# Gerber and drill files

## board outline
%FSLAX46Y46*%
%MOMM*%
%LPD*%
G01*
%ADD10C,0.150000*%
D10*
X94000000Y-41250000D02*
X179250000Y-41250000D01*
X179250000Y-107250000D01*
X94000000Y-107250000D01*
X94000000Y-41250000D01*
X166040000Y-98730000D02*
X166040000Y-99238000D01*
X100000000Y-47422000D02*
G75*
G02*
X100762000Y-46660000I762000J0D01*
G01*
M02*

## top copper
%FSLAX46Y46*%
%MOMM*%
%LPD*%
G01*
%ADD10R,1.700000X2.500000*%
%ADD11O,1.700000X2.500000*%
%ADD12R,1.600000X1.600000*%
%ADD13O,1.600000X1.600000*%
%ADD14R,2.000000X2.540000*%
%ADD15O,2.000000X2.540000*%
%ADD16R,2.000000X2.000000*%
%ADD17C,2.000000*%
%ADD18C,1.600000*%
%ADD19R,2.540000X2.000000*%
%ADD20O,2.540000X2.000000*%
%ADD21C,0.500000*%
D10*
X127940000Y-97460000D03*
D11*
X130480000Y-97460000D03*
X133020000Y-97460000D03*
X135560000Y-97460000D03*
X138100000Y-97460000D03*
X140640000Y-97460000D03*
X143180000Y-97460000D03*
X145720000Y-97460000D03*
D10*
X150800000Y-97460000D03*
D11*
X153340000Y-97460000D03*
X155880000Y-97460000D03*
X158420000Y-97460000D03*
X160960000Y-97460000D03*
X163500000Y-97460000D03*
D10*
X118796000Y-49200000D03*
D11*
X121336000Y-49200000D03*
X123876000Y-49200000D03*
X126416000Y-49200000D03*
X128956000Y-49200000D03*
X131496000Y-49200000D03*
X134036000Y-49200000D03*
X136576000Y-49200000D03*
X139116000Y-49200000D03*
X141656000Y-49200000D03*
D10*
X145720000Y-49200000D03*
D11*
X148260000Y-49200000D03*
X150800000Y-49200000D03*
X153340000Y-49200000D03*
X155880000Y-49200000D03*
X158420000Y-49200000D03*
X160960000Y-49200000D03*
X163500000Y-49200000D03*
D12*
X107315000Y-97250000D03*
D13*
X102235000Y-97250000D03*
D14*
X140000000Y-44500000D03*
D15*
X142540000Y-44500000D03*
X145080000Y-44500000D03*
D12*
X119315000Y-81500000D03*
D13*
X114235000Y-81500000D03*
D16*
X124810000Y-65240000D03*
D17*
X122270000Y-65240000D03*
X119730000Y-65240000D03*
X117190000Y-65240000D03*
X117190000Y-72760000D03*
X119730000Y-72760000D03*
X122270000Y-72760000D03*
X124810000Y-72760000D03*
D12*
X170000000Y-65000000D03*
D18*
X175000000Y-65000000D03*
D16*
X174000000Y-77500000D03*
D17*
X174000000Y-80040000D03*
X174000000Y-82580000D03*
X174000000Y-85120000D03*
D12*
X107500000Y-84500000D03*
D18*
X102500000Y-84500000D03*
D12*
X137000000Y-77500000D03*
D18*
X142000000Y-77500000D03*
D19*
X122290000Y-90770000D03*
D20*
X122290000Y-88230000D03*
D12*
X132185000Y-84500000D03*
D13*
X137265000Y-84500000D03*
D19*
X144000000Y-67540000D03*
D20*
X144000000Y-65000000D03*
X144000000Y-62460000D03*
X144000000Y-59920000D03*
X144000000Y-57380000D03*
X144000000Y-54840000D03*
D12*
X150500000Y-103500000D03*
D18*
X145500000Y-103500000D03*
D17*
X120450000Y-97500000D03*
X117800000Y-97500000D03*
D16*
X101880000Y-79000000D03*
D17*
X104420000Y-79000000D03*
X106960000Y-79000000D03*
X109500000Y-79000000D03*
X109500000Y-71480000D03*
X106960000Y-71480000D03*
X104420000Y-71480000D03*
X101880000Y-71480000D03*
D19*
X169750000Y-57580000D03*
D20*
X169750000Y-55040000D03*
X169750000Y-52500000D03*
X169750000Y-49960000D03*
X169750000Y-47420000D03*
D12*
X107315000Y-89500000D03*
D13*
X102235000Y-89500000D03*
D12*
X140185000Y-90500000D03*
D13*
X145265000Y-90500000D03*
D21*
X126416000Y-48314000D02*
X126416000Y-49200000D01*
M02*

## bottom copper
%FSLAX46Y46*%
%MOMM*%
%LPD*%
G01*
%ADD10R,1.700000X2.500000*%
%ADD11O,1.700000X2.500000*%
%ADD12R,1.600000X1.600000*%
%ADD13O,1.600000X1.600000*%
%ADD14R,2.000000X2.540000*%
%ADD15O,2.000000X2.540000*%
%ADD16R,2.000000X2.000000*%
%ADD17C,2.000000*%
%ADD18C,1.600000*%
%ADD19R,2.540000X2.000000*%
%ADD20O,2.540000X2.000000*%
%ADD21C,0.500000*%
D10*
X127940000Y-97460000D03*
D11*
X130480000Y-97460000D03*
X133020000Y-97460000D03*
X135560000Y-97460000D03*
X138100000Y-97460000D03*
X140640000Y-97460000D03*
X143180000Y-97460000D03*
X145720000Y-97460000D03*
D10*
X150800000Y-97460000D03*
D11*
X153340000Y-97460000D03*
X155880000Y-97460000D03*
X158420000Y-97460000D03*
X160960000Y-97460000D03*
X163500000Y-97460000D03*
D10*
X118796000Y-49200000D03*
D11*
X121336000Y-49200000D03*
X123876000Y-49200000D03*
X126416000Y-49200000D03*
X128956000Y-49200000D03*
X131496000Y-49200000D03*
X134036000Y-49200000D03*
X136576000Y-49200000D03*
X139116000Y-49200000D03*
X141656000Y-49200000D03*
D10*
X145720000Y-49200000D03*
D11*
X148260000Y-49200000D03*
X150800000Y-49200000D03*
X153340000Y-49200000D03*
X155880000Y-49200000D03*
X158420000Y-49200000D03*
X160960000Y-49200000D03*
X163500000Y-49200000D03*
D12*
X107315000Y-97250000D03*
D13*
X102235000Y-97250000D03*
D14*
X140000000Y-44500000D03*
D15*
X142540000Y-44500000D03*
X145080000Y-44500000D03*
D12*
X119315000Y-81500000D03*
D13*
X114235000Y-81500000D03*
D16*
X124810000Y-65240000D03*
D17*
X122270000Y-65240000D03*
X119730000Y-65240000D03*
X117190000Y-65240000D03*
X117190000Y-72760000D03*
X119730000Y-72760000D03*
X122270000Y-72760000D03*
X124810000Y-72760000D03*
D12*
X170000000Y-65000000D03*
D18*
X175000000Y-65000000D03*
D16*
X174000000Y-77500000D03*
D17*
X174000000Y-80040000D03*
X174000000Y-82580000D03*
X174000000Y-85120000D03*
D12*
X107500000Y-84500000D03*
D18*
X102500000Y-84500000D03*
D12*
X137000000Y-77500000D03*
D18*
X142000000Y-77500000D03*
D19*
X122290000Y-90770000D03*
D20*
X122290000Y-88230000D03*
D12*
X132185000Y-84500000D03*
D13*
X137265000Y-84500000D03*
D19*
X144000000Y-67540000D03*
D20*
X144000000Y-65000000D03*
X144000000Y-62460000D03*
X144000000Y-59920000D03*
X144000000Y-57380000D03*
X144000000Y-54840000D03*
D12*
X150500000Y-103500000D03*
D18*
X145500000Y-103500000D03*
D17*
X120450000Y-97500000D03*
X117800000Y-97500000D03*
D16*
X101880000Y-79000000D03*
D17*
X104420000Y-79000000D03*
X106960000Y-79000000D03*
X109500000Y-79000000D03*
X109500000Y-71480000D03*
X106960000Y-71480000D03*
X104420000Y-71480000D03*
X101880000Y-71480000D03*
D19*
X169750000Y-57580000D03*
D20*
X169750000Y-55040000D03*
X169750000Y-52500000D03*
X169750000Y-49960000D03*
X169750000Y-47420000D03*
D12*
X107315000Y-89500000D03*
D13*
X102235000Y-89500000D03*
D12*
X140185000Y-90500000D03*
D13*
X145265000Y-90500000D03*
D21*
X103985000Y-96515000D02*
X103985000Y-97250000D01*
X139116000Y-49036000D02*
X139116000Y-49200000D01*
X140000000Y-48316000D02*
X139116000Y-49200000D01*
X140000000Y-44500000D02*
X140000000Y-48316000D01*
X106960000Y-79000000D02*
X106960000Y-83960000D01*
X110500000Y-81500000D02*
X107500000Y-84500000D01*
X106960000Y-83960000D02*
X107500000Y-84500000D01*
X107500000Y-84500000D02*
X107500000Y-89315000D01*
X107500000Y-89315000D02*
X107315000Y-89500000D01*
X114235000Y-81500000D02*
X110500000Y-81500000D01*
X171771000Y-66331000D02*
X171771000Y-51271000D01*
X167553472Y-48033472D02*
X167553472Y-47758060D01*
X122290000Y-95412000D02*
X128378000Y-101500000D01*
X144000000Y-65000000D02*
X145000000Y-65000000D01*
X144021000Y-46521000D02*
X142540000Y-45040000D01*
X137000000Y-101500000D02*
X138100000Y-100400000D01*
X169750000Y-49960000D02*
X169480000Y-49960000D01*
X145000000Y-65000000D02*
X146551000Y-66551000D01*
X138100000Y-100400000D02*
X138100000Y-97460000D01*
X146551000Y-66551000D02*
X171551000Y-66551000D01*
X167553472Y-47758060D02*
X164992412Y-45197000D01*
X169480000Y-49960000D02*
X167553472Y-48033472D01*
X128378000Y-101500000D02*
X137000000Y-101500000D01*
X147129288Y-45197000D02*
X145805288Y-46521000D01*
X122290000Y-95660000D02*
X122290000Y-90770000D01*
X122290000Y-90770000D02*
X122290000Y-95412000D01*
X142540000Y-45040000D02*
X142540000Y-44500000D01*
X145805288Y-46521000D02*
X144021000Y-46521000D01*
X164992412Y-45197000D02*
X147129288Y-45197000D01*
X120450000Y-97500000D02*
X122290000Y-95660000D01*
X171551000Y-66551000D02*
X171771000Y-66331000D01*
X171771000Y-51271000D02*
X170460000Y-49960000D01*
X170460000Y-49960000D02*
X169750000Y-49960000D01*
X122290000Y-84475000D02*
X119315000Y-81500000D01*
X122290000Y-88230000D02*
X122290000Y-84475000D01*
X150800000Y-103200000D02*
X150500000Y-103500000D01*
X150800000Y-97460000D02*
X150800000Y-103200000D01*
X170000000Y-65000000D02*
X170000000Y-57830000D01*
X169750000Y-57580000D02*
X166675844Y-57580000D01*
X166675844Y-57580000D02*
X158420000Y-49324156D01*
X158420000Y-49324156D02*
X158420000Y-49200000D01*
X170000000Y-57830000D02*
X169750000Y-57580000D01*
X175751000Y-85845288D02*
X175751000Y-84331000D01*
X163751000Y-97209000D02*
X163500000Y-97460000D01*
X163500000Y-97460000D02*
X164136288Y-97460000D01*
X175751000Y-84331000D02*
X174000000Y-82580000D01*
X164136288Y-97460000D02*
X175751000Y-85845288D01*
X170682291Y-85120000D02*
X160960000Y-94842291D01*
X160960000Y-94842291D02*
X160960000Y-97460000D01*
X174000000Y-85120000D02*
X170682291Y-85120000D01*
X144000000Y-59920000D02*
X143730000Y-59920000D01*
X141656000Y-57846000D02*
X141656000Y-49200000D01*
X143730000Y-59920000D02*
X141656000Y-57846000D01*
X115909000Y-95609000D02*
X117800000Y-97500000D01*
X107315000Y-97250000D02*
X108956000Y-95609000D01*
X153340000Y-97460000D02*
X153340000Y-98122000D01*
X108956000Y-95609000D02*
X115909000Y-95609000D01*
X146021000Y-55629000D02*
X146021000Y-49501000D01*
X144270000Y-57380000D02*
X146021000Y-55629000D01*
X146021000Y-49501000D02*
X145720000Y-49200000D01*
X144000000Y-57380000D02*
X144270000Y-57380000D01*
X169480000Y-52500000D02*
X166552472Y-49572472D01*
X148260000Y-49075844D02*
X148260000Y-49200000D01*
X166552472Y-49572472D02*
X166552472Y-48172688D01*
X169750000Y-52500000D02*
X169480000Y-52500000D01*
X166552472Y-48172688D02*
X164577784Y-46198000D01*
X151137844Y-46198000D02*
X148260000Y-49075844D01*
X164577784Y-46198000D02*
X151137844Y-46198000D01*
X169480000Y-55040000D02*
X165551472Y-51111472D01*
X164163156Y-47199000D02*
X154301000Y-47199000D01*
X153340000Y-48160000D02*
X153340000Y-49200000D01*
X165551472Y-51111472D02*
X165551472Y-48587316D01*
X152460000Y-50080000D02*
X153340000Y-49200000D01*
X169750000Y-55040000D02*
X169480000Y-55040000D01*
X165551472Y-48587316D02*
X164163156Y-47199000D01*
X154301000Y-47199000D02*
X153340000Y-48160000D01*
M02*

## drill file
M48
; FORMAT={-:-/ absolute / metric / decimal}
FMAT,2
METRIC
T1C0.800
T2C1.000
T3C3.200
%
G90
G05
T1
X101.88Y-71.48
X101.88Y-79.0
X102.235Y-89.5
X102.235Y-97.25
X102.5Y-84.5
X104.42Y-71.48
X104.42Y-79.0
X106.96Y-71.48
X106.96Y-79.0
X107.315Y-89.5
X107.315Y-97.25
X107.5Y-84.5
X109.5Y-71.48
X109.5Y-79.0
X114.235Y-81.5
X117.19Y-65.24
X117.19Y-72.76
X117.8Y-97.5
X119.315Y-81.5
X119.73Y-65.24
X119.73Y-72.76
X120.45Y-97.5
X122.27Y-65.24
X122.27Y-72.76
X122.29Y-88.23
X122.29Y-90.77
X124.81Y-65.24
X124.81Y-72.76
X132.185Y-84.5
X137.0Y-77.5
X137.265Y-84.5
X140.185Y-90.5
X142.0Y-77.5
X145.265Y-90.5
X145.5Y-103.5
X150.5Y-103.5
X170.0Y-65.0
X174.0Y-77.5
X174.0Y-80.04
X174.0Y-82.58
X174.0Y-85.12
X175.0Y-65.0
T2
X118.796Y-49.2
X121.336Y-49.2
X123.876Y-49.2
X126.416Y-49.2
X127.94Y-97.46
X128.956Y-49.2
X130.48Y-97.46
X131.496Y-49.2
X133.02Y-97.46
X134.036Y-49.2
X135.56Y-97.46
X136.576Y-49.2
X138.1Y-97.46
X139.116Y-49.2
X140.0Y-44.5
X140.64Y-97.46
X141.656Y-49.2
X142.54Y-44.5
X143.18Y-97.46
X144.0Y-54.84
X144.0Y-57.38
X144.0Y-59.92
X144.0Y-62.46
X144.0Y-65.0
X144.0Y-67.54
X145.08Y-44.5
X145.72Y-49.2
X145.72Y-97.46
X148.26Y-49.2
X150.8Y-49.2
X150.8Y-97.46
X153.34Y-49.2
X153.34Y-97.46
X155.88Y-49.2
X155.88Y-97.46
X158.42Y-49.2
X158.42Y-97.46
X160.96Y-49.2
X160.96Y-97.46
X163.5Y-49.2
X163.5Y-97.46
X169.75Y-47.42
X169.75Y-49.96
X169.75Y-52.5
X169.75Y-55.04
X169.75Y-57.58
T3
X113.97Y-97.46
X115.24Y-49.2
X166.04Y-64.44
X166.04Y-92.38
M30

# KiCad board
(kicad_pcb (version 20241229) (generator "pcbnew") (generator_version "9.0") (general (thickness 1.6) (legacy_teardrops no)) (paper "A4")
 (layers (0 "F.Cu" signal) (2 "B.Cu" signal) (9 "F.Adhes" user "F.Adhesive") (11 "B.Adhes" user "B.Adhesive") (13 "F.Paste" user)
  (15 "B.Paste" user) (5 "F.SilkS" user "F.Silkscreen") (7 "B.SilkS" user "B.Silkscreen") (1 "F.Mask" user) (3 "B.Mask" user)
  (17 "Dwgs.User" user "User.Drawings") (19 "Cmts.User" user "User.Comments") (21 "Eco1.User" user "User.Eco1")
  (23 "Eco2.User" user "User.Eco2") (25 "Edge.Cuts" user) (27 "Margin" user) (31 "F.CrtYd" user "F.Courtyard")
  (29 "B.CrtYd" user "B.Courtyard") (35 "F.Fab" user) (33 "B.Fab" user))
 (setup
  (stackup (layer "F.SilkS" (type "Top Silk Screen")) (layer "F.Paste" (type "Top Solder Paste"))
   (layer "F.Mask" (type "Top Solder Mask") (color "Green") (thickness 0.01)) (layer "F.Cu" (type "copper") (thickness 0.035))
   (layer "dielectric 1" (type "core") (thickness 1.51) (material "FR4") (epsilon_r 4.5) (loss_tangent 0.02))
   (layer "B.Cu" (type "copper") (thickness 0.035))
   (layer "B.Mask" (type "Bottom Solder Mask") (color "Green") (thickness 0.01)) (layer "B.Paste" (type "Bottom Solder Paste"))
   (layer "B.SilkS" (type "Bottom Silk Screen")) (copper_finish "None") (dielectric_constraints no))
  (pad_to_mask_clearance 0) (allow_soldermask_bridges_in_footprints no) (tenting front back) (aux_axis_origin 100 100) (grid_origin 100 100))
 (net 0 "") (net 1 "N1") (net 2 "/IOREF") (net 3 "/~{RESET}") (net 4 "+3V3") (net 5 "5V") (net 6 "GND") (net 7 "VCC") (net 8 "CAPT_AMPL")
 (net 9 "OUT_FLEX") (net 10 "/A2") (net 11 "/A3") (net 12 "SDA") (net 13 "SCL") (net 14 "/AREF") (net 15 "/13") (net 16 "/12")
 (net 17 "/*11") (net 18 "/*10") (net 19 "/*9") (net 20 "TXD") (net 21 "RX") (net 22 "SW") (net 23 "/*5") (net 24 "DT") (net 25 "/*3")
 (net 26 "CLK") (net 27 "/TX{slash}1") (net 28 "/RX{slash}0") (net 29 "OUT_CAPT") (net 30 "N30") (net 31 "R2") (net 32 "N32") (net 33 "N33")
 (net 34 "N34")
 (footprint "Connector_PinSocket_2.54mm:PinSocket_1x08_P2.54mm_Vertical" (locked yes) (layer "F.Cu") (at 127.94 97.46 90)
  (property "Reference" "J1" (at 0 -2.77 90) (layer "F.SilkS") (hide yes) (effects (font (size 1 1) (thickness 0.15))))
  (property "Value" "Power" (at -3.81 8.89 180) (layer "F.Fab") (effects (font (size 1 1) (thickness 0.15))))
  (pad "1" thru_hole rect (at 0 0 90) (size 2.5 1.7) (drill 1) (layers "*.Cu" "*.Mask") (remove_unused_layers no) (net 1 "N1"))
  (pad "2" thru_hole oval (at 0 2.54 90) (size 2.5 1.7) (drill 1) (layers "*.Cu" "*.Mask") (remove_unused_layers no) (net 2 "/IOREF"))
  (pad "3" thru_hole oval (at 0 5.08 90) (size 2.5 1.7) (drill 1) (layers "*.Cu" "*.Mask") (remove_unused_layers no) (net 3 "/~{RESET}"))
  (pad "4" thru_hole oval (at 0 7.62 90) (size 2.5 1.7) (drill 1) (layers "*.Cu" "*.Mask") (remove_unused_layers no) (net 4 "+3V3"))
  (pad "5" thru_hole oval (at 0 10.16 90) (size 2.5 1.7) (drill 1) (layers "*.Cu" "*.Mask") (remove_unused_layers no) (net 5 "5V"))
  (pad "6" thru_hole oval (at 0 12.7 90) (size 2.5 1.7) (drill 1) (layers "*.Cu" "*.Mask") (remove_unused_layers no) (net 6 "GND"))
  (pad "7" thru_hole oval (at 0 15.24 90) (size 2.5 1.7) (drill 1) (layers "*.Cu" "*.Mask") (remove_unused_layers no) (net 6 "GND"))
  (pad "8" thru_hole oval (at 0 17.78 90) (size 2.5 1.7) (drill 1) (layers "*.Cu" "*.Mask") (remove_unused_layers no) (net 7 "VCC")))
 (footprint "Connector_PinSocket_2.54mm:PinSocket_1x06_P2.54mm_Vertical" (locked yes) (layer "F.Cu") (at 150.8 97.46 90)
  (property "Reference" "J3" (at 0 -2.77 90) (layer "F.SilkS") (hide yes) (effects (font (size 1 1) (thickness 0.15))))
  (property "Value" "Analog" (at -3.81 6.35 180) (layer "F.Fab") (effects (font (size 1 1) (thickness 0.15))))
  (pad "1" thru_hole rect (at 0 0 90) (size 2.5 1.7) (drill 1) (layers "*.Cu" "*.Mask") (remove_unused_layers no) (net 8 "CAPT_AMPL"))
  (pad "2" thru_hole oval (at 0 2.54 90) (size 2.5 1.7) (drill 1) (layers "*.Cu" "*.Mask") (remove_unused_layers no) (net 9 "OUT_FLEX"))
  (pad "3" thru_hole oval (at 0 5.08 90) (size 2.5 1.7) (drill 1) (layers "*.Cu" "*.Mask") (remove_unused_layers no) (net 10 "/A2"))
  (pad "4" thru_hole oval (at 0 7.62 90) (size 2.5 1.7) (drill 1) (layers "*.Cu" "*.Mask") (remove_unused_layers no) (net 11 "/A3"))
  (pad "5" thru_hole oval (at 0 10.16 90) (size 2.5 1.7) (drill 1) (layers "*.Cu" "*.Mask") (remove_unused_layers no) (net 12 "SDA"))
  (pad "6" thru_hole oval (at 0 12.7 90) (size 2.5 1.7) (drill 1) (layers "*.Cu" "*.Mask") (remove_unused_layers no) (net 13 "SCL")))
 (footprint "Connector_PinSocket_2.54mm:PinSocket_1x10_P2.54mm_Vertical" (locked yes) (layer "F.Cu") (at 118.796 49.2 90)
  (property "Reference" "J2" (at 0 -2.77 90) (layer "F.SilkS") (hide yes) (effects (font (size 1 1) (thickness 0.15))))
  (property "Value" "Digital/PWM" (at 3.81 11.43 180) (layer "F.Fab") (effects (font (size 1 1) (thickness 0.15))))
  (pad "1" thru_hole rect (at 0 0 90) (size 2.5 1.7) (drill 1) (layers "*.Cu" "*.Mask") (remove_unused_layers no) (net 13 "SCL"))
  (pad "2" thru_hole oval (at 0 2.54 90) (size 2.5 1.7) (drill 1) (layers "*.Cu" "*.Mask") (remove_unused_layers no) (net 12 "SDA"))
  (pad "3" thru_hole oval (at 0 5.08 90) (size 2.5 1.7) (drill 1) (layers "*.Cu" "*.Mask") (remove_unused_layers no) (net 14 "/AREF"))
  (pad "4" thru_hole oval (at 0 7.62 90) (size 2.5 1.7) (drill 1) (layers "*.Cu" "*.Mask") (remove_unused_layers no) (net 6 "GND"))
  (pad "5" thru_hole oval (at 0 10.16 90) (size 2.5 1.7) (drill 1) (layers "*.Cu" "*.Mask") (remove_unused_layers no) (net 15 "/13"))
  (pad "6" thru_hole oval (at 0 12.7 90) (size 2.5 1.7) (drill 1) (layers "*.Cu" "*.Mask") (remove_unused_layers no) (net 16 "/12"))
  (pad "7" thru_hole oval (at 0 15.24 90) (size 2.5 1.7) (drill 1) (layers "*.Cu" "*.Mask") (remove_unused_layers no) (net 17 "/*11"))
  (pad "8" thru_hole oval (at 0 17.78 90) (size 2.5 1.7) (drill 1) (layers "*.Cu" "*.Mask") (remove_unused_layers no) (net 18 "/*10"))
  (pad "9" thru_hole oval (at 0 20.32 90) (size 2.5 1.7) (drill 1) (layers "*.Cu" "*.Mask") (remove_unused_layers no) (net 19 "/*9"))
  (pad "10" thru_hole oval (at 0 22.86 90) (size 2.5 1.7) (drill 1) (layers "*.Cu" "*.Mask") (remove_unused_layers no) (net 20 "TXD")))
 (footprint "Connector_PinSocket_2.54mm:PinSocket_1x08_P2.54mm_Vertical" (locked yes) (layer "F.Cu") (at 145.72 49.2 90)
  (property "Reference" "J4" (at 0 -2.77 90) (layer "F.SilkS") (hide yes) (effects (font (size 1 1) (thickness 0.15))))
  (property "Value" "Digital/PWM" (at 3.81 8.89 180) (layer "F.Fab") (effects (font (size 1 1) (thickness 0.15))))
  (pad "1" thru_hole rect (at 0 0 90) (size 2.5 1.7) (drill 1) (layers "*.Cu" "*.Mask") (remove_unused_layers no) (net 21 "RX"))
  (pad "2" thru_hole oval (at 0 2.54 90) (size 2.5 1.7) (drill 1) (layers "*.Cu" "*.Mask") (remove_unused_layers no) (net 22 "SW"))
  (pad "3" thru_hole oval (at 0 5.08 90) (size 2.5 1.7) (drill 1) (layers "*.Cu" "*.Mask") (remove_unused_layers no) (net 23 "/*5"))
  (pad "4" thru_hole oval (at 0 7.62 90) (size 2.5 1.7) (drill 1) (layers "*.Cu" "*.Mask") (remove_unused_layers no) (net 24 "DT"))
  (pad "5" thru_hole oval (at 0 10.16 90) (size 2.5 1.7) (drill 1) (layers "*.Cu" "*.Mask") (remove_unused_layers no) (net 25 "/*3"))
  (pad "6" thru_hole oval (at 0 12.7 90) (size 2.5 1.7) (drill 1) (layers "*.Cu" "*.Mask") (remove_unused_layers no) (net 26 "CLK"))
  (pad "7" thru_hole oval (at 0 15.24 90) (size 2.5 1.7) (drill 1) (layers "*.Cu" "*.Mask") (remove_unused_layers no) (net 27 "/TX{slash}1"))
  (pad "8" thru_hole oval (at 0 17.78 90) (size 2.5 1.7) (drill 1) (layers "*.Cu" "*.Mask") (remove_unused_layers no) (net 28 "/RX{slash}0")))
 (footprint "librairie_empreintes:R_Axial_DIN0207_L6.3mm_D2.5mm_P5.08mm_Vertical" (layer "F.Cu") (at 107.315 97.25 180)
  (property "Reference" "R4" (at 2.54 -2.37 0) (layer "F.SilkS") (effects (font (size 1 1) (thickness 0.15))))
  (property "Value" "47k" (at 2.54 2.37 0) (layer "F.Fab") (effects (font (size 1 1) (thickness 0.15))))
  (pad "1" thru_hole rect (at 0 0 180) (size 1.6 1.6) (drill 0.8) (layers "*.Cu" "*.Mask") (remove_unused_layers no) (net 9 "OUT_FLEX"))
  (pad "2" thru_hole oval (at 5.08 0 180) (size 1.6 1.6) (drill 0.8) (layers "*.Cu" "*.Mask") (remove_unused_layers no) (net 6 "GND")))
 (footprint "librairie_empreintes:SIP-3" (layer "F.Cu") (at 142.54 44.5)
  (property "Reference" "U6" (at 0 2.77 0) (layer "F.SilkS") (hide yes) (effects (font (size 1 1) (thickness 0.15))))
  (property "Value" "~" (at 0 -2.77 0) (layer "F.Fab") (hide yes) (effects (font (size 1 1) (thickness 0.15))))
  (pad "1" thru_hole rect (at -2.54 0) (size 2 2.54) (drill 1) (layers "*.Cu" "*.Mask") (remove_unused_layers no) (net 19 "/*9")
   (thermal_bridge_angle 45))
  (pad "2" thru_hole oval (at 0 0) (size 2 2.54) (drill 1) (layers "*.Cu" "*.Mask") (remove_unused_layers no) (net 5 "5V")
   (thermal_bridge_angle 45))
  (pad "3" thru_hole oval (at 2.54 0) (size 2 2.54) (drill 1) (layers "*.Cu" "*.Mask") (remove_unused_layers no) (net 6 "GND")
   (thermal_bridge_angle 45)))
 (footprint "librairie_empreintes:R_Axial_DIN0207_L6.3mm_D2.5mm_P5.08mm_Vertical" (layer "F.Cu") (at 119.315 81.5 180)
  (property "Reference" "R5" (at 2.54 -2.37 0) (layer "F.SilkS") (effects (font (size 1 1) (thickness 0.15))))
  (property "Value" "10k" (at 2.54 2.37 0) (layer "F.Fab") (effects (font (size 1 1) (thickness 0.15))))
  (pad "1" thru_hole rect (at 0 0 180) (size 1.6 1.6) (drill 0.8) (layers "*.Cu" "*.Mask") (remove_unused_layers no) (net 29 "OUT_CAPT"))
  (pad "2" thru_hole oval (at 5.08 0 180) (size 1.6 1.6) (drill 0.8) (layers "*.Cu" "*.Mask") (remove_unused_layers no) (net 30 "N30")))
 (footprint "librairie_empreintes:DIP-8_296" (layer "F.Cu") (at 121 69 180)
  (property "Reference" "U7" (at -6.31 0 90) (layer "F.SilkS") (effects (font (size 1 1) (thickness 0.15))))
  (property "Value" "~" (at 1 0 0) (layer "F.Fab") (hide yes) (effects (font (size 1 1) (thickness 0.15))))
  (pad "1" thru_hole rect (at -3.81 3.76 180) (size 2 2) (drill 0.8) (layers "*.Cu" "*.Mask") (remove_unused_layers no) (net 18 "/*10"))
  (pad "2" thru_hole circle (at -1.27 3.76 180) (size 2 2) (drill 0.8) (layers "*.Cu" "*.Mask") (remove_unused_layers no) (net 15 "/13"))
  (pad "3" thru_hole circle (at 1.27 3.76 180) (size 2 2) (drill 0.8) (layers "*.Cu" "*.Mask") (remove_unused_layers no) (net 17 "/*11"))
  (pad "4" thru_hole circle (at 3.81 3.76 180) (size 2 2) (drill 0.8) (layers "*.Cu" "*.Mask") (remove_unused_layers no) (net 6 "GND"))
  (pad "5" thru_hole circle (at 3.81 -3.76 180) (size 2 2) (drill 0.8) (layers "*.Cu" "*.Mask") (remove_unused_layers no) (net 6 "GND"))
  (pad "6" thru_hole circle (at 1.27 -3.76 180) (size 2 2) (drill 0.8) (layers "*.Cu" "*.Mask") (remove_unused_layers no) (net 6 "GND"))
  (pad "7" thru_hole circle (at -1.27 -3.76 180) (size 2 2) (drill 0.8) (layers "*.Cu" "*.Mask") (remove_unused_layers no) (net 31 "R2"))
  (pad "8" thru_hole circle (at -3.81 -3.76 180) (size 2 2) (drill 0.8) (layers "*.Cu" "*.Mask") (remove_unused_layers no) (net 5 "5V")))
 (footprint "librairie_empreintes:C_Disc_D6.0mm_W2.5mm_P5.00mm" (layer "F.Cu") (at 170 65)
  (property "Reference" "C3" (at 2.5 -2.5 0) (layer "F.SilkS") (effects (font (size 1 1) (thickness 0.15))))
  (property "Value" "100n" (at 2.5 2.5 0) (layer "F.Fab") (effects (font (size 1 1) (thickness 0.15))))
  (pad "1" thru_hole rect (at 0 0) (size 1.6 1.6) (drill 0.8) (layers "*.Cu" "*.Mask") (remove_unused_layers no) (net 26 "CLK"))
  (pad "2" thru_hole circle (at 5 0) (size 1.6 1.6) (drill 0.8) (layers "*.Cu" "*.Mask") (remove_unused_layers no) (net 6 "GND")))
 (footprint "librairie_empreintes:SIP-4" (layer "F.Cu") (at 174 81.31 -90)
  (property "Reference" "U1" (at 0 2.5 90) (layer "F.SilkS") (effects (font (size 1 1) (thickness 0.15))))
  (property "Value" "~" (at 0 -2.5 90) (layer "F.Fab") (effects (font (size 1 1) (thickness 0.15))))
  (pad "1" thru_hole rect (at -3.81 0 270) (size 2 2) (drill 0.8) (layers "*.Cu" "*.Mask") (remove_unused_layers no) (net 6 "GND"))
  (pad "2" thru_hole circle (at -1.27 0 270) (size 2 2) (drill 0.8) (layers "*.Cu" "*.Mask") (remove_unused_layers no) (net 5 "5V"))
  (pad "3" thru_hole circle (at 1.27 0 270) (size 2 2) (drill 0.8) (layers "*.Cu" "*.Mask") (remove_unused_layers no) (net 13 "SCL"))
  (pad "4" thru_hole circle (at 3.81 0 270) (size 2 2) (drill 0.8) (layers "*.Cu" "*.Mask") (remove_unused_layers no) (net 12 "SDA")))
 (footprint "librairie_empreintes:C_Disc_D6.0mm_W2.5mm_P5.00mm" (layer "F.Cu") (at 107.5 84.5 180)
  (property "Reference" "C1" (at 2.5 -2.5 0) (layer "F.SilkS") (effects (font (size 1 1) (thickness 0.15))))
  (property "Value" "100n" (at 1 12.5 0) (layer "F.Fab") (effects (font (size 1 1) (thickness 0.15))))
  (pad "1" thru_hole rect (at 0 0 180) (size 1.6 1.6) (drill 0.8) (layers "*.Cu" "*.Mask") (remove_unused_layers no) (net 30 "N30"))
  (pad "2" thru_hole circle (at 5 0 180) (size 1.6 1.6) (drill 0.8) (layers "*.Cu" "*.Mask") (remove_unused_layers no) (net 6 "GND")))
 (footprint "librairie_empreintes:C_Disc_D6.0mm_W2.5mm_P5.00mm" (layer "F.Cu") (at 137 77.5)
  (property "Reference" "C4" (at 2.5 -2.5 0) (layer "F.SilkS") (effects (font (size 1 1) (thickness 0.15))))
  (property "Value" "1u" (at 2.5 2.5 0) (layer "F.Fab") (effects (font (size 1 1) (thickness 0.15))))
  (pad "1" thru_hole rect (at 0 0) (size 1.6 1.6) (drill 0.8) (layers "*.Cu" "*.Mask") (remove_unused_layers no) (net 31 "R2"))
  (pad "2" thru_hole circle (at 5 0) (size 1.6 1.6) (drill 0.8) (layers "*.Cu" "*.Mask") (remove_unused_layers no) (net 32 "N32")))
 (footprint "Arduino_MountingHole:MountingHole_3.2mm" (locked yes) (layer "F.Cu") (at 115.24 49.2)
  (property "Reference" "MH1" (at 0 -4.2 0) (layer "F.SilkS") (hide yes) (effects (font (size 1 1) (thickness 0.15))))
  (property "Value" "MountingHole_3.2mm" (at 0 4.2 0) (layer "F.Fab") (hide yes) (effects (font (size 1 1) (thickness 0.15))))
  (pad "" np_thru_hole circle (at 0 0) (size 3.2 3.2) (drill 3.2) (layers "*.Cu" "*.Mask")))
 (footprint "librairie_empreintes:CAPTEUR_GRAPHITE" (layer "F.Cu") (at 128.29 88.73 90)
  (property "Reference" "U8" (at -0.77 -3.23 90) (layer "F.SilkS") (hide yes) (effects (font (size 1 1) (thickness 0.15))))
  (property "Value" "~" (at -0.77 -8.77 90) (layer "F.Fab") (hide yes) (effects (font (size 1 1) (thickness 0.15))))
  (pad "1" thru_hole rect (at -2.04 -6 90) (size 2 2.54) (drill 0.8) (layers "*.Cu" "*.Mask") (remove_unused_layers no) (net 5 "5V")
   (thermal_bridge_angle 45))
  (pad "2" thru_hole oval (at 0.5 -6 90) (size 2 2.54) (drill 0.8) (layers "*.Cu" "*.Mask") (remove_unused_layers no) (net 29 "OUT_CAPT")
   (thermal_bridge_angle 45)))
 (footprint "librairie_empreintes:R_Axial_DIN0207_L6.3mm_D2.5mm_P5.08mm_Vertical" (layer "F.Cu") (at 132.185 84.5)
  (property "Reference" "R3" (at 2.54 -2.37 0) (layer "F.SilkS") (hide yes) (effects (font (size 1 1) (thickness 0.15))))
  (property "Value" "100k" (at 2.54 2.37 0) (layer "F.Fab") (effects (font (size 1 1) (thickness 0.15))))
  (pad "1" thru_hole rect (at 0 0) (size 1.6 1.6) (drill 0.8) (layers "*.Cu" "*.Mask") (remove_unused_layers no) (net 31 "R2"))
  (pad "2" thru_hole oval (at 5.08 0) (size 1.6 1.6) (drill 0.8) (layers "*.Cu" "*.Mask") (remove_unused_layers no) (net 32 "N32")))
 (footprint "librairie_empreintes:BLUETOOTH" (layer "F.Cu") (at 144 61.19 90)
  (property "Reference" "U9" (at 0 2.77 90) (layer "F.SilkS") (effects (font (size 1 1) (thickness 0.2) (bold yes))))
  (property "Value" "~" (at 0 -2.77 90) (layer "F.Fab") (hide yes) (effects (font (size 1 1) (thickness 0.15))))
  (pad "1" thru_hole rect (at -6.35 0 90) (size 2 2.54) (drill 1) (layers "*.Cu" "*.Mask") (remove_unused_layers no) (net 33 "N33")
   (thermal_bridge_angle 45))
  (pad "2" thru_hole oval (at -3.81 0 90) (size 2 2.54) (drill 1) (layers "*.Cu" "*.Mask") (remove_unused_layers no) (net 5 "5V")
   (thermal_bridge_angle 45))
  (pad "3" thru_hole oval (at -1.27 0 90) (size 2 2.54) (drill 1) (layers "*.Cu" "*.Mask") (remove_unused_layers no) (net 6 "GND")
   (thermal_bridge_angle 45))
  (pad "4" thru_hole oval (at 1.27 0 90) (size 2 2.54) (drill 1) (layers "*.Cu" "*.Mask") (remove_unused_layers no) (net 20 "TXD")
   (thermal_bridge_angle 45))
  (pad "5" thru_hole oval (at 3.81 0 90) (size 2 2.54) (drill 1) (layers "*.Cu" "*.Mask") (remove_unused_layers no) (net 21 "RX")
   (thermal_bridge_angle 45))
  (pad "6" thru_hole oval (at 6.35 0 90) (size 2 2.54) (drill 1) (layers "*.Cu" "*.Mask") (remove_unused_layers no) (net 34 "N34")
   (thermal_bridge_angle 45)))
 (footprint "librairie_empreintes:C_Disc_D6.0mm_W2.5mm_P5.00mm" (layer "F.Cu") (at 150.5 103.5 180)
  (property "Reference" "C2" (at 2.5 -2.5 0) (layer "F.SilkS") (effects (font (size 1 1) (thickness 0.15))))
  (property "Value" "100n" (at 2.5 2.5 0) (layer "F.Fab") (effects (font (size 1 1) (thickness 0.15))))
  (pad "1" thru_hole rect (at 0 0 180) (size 1.6 1.6) (drill 0.8) (layers "*.Cu" "*.Mask") (remove_unused_layers no) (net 8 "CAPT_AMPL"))
  (pad "2" thru_hole circle (at 5 0 180) (size 1.6 1.6) (drill 0.8) (layers "*.Cu" "*.Mask") (remove_unused_layers no) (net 6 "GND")))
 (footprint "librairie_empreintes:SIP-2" (layer "F.Cu") (at 119 96.75 180)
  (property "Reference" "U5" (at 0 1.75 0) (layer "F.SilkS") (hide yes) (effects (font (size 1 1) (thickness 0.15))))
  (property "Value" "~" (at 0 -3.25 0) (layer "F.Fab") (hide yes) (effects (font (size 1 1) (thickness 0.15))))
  (pad "1" thru_hole circle (at -1.45 -0.75 180) (size 2 2) (drill 0.8) (layers "*.Cu" "*.Mask") (remove_unused_layers no) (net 5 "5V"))
  (pad "2" thru_hole circle (at 1.2 -0.75 180) (size 2 2) (drill 0.8) (layers "*.Cu" "*.Mask") (remove_unused_layers no) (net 9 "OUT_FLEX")))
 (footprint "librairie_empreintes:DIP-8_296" (layer "F.Cu") (at 105.69 75.24)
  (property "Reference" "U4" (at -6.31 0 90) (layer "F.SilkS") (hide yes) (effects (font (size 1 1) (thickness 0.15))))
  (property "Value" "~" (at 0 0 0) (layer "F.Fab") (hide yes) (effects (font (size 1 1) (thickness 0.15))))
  (pad "1" thru_hole rect (at -3.81 3.76) (size 2 2) (drill 0.8) (layers "*.Cu" "*.Mask") (remove_unused_layers no))
  (pad "2" thru_hole circle (at -1.27 3.76) (size 2 2) (drill 0.8) (layers "*.Cu" "*.Mask") (remove_unused_layers no) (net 31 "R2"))
  (pad "3" thru_hole circle (at 1.27 3.76) (size 2 2) (drill 0.8) (layers "*.Cu" "*.Mask") (remove_unused_layers no) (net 30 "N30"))
  (pad "4" thru_hole circle (at 3.81 3.76) (size 2 2) (drill 0.8) (layers "*.Cu" "*.Mask") (remove_unused_layers no) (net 6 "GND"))
  (pad "5" thru_hole circle (at 3.81 -3.76) (size 2 2) (drill 0.8) (layers "*.Cu" "*.Mask") (remove_unused_layers no))
  (pad "6" thru_hole circle (at 1.27 -3.76) (size 2 2) (drill 0.8) (layers "*.Cu" "*.Mask") (remove_unused_layers no) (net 32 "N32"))
  (pad "7" thru_hole circle (at -1.27 -3.76) (size 2 2) (drill 0.8) (layers "*.Cu" "*.Mask") (remove_unused_layers no) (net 5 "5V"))
  (pad "8" thru_hole circle (at -3.81 -3.76) (size 2 2) (drill 0.8) (layers "*.Cu" "*.Mask") (remove_unused_layers no)))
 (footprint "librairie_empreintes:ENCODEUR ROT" (layer "F.Cu") (at 169.75 52.5 90)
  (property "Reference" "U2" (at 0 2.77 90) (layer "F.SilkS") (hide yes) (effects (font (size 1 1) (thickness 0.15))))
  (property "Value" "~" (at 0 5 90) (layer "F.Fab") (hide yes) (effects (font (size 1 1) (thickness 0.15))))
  (pad "1" thru_hole rect (at -5.08 0 90) (size 2 2.54) (drill 1) (layers "*.Cu" "*.Mask") (remove_unused_layers no) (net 26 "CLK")
   (thermal_bridge_angle 45))
  (pad "2" thru_hole oval (at -2.54 0 90) (size 2 2.54) (drill 1) (layers "*.Cu" "*.Mask") (remove_unused_layers no) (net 24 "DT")
   (thermal_bridge_angle 45))
  (pad "3" thru_hole oval (at 0 0 90) (size 2 2.54) (drill 1) (layers "*.Cu" "*.Mask") (remove_unused_layers no) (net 22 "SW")
   (thermal_bridge_angle 45))
  (pad "4" thru_hole oval (at 2.54 0 90) (size 2 2.54) (drill 1) (layers "*.Cu" "*.Mask") (remove_unused_layers no) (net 5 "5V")
   (thermal_bridge_angle 45))
  (pad "5" thru_hole oval (at 5.08 0 90) (size 2 2.54) (drill 1) (layers "*.Cu" "*.Mask") (remove_unused_layers no) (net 6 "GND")
   (thermal_bridge_angle 45)))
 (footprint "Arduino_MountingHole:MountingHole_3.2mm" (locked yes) (layer "F.Cu") (at 113.97 97.46)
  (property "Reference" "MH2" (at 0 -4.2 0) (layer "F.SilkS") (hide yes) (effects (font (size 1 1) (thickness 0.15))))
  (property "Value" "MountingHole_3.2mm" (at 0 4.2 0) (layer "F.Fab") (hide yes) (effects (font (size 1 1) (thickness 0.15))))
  (pad "" np_thru_hole circle (at 0 0) (size 3.2 3.2) (drill 3.2) (layers "*.Cu" "*.Mask")))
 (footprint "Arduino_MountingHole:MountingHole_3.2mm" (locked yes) (layer "F.Cu") (at 166.04 64.44)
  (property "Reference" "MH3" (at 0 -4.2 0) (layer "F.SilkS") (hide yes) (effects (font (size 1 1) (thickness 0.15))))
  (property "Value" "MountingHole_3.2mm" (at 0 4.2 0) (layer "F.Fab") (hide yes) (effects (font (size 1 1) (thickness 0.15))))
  (pad "" np_thru_hole circle (at 0 0) (size 3.2 3.2) (drill 3.2) (layers "*.Cu" "*.Mask")))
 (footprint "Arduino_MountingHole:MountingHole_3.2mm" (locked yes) (layer "F.Cu") (at 166.04 92.38)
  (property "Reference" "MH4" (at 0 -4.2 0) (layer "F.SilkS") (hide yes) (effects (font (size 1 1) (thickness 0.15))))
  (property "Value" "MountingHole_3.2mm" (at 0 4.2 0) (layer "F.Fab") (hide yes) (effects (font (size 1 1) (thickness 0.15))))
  (pad "" np_thru_hole circle (at 0 0) (size 3.2 3.2) (drill 3.2) (layers "*.Cu" "*.Mask")))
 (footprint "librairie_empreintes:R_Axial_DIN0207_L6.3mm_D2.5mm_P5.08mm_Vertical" (layer "F.Cu") (at 107.315 89.5 180)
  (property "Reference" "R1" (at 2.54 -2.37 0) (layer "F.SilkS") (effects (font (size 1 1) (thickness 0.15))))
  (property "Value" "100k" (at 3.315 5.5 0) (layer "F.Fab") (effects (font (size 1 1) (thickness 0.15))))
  (pad "1" thru_hole rect (at 0 0 180) (size 1.6 1.6) (drill 0.8) (layers "*.Cu" "*.Mask") (remove_unused_layers no) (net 30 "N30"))
  (pad "2" thru_hole oval (at 5.08 0 180) (size 1.6 1.6) (drill 0.8) (layers "*.Cu" "*.Mask") (remove_unused_layers no) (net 6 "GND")))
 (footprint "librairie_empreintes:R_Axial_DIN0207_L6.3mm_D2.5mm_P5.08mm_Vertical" (layer "F.Cu") (at 140.185 90.5)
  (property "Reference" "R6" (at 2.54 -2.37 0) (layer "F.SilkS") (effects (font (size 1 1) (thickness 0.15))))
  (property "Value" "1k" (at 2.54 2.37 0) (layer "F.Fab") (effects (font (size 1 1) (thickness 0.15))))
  (pad "1" thru_hole rect (at 0 0) (size 1.6 1.6) (drill 0.8) (layers "*.Cu" "*.Mask") (remove_unused_layers no) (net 32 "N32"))
  (pad "2" thru_hole oval (at 5.08 0) (size 1.6 1.6) (drill 0.8) (layers "*.Cu" "*.Mask") (remove_unused_layers no) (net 8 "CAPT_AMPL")))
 (gr_rect (start 94 41.25) (end 179.25 107.25) (stroke (width 0.15) (type solid)) (fill no) (layer "Edge.Cuts"))
 (gr_line (start 166.04 98.73) (end 166.04 99.238) (stroke (width 0.15) (type solid)) (layer "Edge.Cuts"))
 (gr_arc (start 100 47.422) (mid 100.223185 46.883185) (end 100.762 46.66) (stroke (width 0.15) (type solid)) (layer "Edge.Cuts"))
 (segment (start 126.416 48.314) (end 126.416 49.2) (width 0.5) (layer "F.Cu") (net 6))
 (segment (start 103.985 96.515) (end 103.985 97.25) (width 0.5) (layer "B.Cu") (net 6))
 (segment (start 139.116 49.036) (end 139.116 49.2) (width 0.5) (layer "B.Cu") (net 19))
 (segment (start 140 48.316) (end 139.116 49.2) (width 0.5) (layer "B.Cu") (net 19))
 (segment (start 140 44.5) (end 140 48.316) (width 0.5) (layer "B.Cu") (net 19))
 (segment (start 106.96 79) (end 106.96 83.96) (width 0.5) (layer "B.Cu") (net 30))
 (segment (start 110.5 81.5) (end 107.5 84.5) (width 0.5) (layer "B.Cu") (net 30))
 (segment (start 106.96 83.96) (end 107.5 84.5) (width 0.5) (layer "B.Cu") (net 30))
 (segment (start 107.5 84.5) (end 107.5 89.315) (width 0.5) (layer "B.Cu") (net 30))
 (segment (start 107.5 89.315) (end 107.315 89.5) (width 0.5) (layer "B.Cu") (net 30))
 (segment (start 114.235 81.5) (end 110.5 81.5) (width 0.5) (layer "B.Cu") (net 30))
 (segment (start 171.771 66.331) (end 171.771 51.271) (width 0.5) (layer "B.Cu") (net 5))
 (segment (start 167.553472 48.033472) (end 167.553472 47.75806) (width 0.5) (layer "B.Cu") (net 5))
 (segment (start 122.29 95.412) (end 128.378 101.5) (width 0.5) (layer "B.Cu") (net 5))
 (segment (start 144 65) (end 145 65) (width 0.5) (layer "B.Cu") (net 5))
 (segment (start 144.021 46.521) (end 142.54 45.04) (width 0.5) (layer "B.Cu") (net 5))
 (segment (start 137 101.5) (end 138.1 100.4) (width 0.5) (layer "B.Cu") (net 5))
 (segment (start 169.75 49.96) (end 169.48 49.96) (width 0.5) (layer "B.Cu") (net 5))
 (segment (start 145 65) (end 146.551 66.551) (width 0.5) (layer "B.Cu") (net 5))
 (segment (start 138.1 100.4) (end 138.1 97.46) (width 0.5) (layer "B.Cu") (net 5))
 (segment (start 146.551 66.551) (end 171.551 66.551) (width 0.5) (layer "B.Cu") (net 5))
 (segment (start 167.553472 47.75806) (end 164.992412 45.197) (width 0.5) (layer "B.Cu") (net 5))
 (segment (start 169.48 49.96) (end 167.553472 48.033472) (width 0.5) (layer "B.Cu") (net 5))
 (segment (start 128.378 101.5) (end 137 101.5) (width 0.5) (layer "B.Cu") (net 5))
 (segment (start 147.129288 45.197) (end 145.805288 46.521) (width 0.5) (layer "B.Cu") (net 5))
 (segment (start 122.29 95.66) (end 122.29 90.77) (width 0.5) (layer "B.Cu") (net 5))
 (segment (start 122.29 90.77) (end 122.29 95.412) (width 0.5) (layer "B.Cu") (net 5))
 (segment (start 142.54 45.04) (end 142.54 44.5) (width 0.5) (layer "B.Cu") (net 5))
 (segment (start 145.805288 46.521) (end 144.021 46.521) (width 0.5) (layer "B.Cu") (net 5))
 (segment (start 164.992412 45.197) (end 147.129288 45.197) (width 0.5) (layer "B.Cu") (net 5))
 (segment (start 120.45 97.5) (end 122.29 95.66) (width 0.5) (layer "B.Cu") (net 5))
 (segment (start 171.551 66.551) (end 171.771 66.331) (width 0.5) (layer "B.Cu") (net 5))
 (segment (start 171.771 51.271) (end 170.46 49.96) (width 0.5) (layer "B.Cu") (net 5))
 (segment (start 170.46 49.96) (end 169.75 49.96) (width 0.5) (layer "B.Cu") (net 5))
 (segment (start 122.29 84.475) (end 119.315 81.5) (width 0.5) (layer "B.Cu") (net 29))
 (segment (start 122.29 88.23) (end 122.29 84.475) (width 0.5) (layer "B.Cu") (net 29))
 (segment (start 150.8 103.2) (end 150.5 103.5) (width 0.5) (layer "B.Cu") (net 8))
 (segment (start 150.8 97.46) (end 150.8 103.2) (width 0.5) (layer "B.Cu") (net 8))
 (segment (start 170 65) (end 170 57.83) (width 0.5) (layer "B.Cu") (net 26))
 (segment (start 169.75 57.58) (end 166.675844 57.58) (width 0.5) (layer "B.Cu") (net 26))
 (segment (start 166.675844 57.58) (end 158.42 49.324156) (width 0.5) (layer "B.Cu") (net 26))
 (segment (start 158.42 49.324156) (end 158.42 49.2) (width 0.5) (layer "B.Cu") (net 26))
 (segment (start 170 57.83) (end 169.75 57.58) (width 0.5) (layer "B.Cu") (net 26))
 (segment (start 175.751 85.845288) (end 175.751 84.331) (width 0.5) (layer "B.Cu") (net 13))
 (segment (start 163.751 97.209) (end 163.5 97.46) (width 0.5) (layer "B.Cu") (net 13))
 (segment (start 163.5 97.46) (end 164.136288 97.46) (width 0.5) (layer "B.Cu") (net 13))
 (segment (start 175.751 84.331) (end 174 82.58) (width 0.5) (layer "B.Cu") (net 13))
 (segment (start 164.136288 97.46) (end 175.751 85.845288) (width 0.5) (layer "B.Cu") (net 13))
 (segment (start 170.682291 85.12) (end 160.96 94.842291) (width 0.5) (layer "B.Cu") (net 12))
 (segment (start 160.96 94.842291) (end 160.96 97.46) (width 0.5) (layer "B.Cu") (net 12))
 (segment (start 174 85.12) (end 170.682291 85.12) (width 0.5) (layer "B.Cu") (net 12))
 (segment (start 144 59.92) (end 143.73 59.92) (width 0.5) (layer "B.Cu") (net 20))
 (segment (start 141.656 57.846) (end 141.656 49.2) (width 0.5) (layer "B.Cu") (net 20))
 (segment (start 143.73 59.92) (end 141.656 57.846) (width 0.5) (layer "B.Cu") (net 20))
 (segment (start 115.909 95.609) (end 117.8 97.5) (width 0.5) (layer "B.Cu") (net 9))
 (segment (start 107.315 97.25) (end 108.956 95.609) (width 0.5) (layer "B.Cu") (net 9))
 (segment (start 153.34 97.46) (end 153.34 98.122) (width 0.5) (layer "B.Cu") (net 9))
 (segment (start 108.956 95.609) (end 115.909 95.609) (width 0.5) (layer "B.Cu") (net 9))
 (segment (start 146.021 55.629) (end 146.021 49.501) (width 0.5) (layer "B.Cu") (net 21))
 (segment (start 144.27 57.38) (end 146.021 55.629) (width 0.5) (layer "B.Cu") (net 21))
 (segment (start 146.021 49.501) (end 145.72 49.2) (width 0.5) (layer "B.Cu") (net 21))
 (segment (start 144 57.38) (end 144.27 57.38) (width 0.5) (layer "B.Cu") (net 21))
 (segment (start 169.48 52.5) (end 166.552472 49.572472) (width 0.5) (layer "B.Cu") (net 22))
 (segment (start 148.26 49.075844) (end 148.26 49.2) (width 0.5) (layer "B.Cu") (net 22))
 (segment (start 166.552472 49.572472) (end 166.552472 48.172688) (width 0.5) (layer "B.Cu") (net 22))
 (segment (start 169.75 52.5) (end 169.48 52.5) (width 0.5) (layer "B.Cu") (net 22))
 (segment (start 166.552472 48.172688) (end 164.577784 46.198) (width 0.5) (layer "B.Cu") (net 22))
 (segment (start 151.137844 46.198) (end 148.26 49.075844) (width 0.5) (layer "B.Cu") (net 22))
 (segment (start 164.577784 46.198) (end 151.137844 46.198) (width 0.5) (layer "B.Cu") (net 22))
 (segment (start 169.48 55.04) (end 165.551472 51.111472) (width 0.5) (layer "B.Cu") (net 24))
 (segment (start 164.163156 47.199) (end 154.301 47.199) (width 0.5) (layer "B.Cu") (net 24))
 (segment (start 153.34 48.16) (end 153.34 49.2) (width 0.5) (layer "B.Cu") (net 24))
 (segment (start 165.551472 51.111472) (end 165.551472 48.587316) (width 0.5) (layer "B.Cu") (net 24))
 (segment (start 152.46 50.08) (end 153.34 49.2) (width 0.5) (layer "B.Cu") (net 24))
 (segment (start 169.75 55.04) (end 169.48 55.04) (width 0.5) (layer "B.Cu") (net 24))
 (segment (start 165.551472 48.587316) (end 164.163156 47.199) (width 0.5) (layer "B.Cu") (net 24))
 (segment (start 154.301 47.199) (end 153.34 48.16) (width 0.5) (layer "B.Cu") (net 24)))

